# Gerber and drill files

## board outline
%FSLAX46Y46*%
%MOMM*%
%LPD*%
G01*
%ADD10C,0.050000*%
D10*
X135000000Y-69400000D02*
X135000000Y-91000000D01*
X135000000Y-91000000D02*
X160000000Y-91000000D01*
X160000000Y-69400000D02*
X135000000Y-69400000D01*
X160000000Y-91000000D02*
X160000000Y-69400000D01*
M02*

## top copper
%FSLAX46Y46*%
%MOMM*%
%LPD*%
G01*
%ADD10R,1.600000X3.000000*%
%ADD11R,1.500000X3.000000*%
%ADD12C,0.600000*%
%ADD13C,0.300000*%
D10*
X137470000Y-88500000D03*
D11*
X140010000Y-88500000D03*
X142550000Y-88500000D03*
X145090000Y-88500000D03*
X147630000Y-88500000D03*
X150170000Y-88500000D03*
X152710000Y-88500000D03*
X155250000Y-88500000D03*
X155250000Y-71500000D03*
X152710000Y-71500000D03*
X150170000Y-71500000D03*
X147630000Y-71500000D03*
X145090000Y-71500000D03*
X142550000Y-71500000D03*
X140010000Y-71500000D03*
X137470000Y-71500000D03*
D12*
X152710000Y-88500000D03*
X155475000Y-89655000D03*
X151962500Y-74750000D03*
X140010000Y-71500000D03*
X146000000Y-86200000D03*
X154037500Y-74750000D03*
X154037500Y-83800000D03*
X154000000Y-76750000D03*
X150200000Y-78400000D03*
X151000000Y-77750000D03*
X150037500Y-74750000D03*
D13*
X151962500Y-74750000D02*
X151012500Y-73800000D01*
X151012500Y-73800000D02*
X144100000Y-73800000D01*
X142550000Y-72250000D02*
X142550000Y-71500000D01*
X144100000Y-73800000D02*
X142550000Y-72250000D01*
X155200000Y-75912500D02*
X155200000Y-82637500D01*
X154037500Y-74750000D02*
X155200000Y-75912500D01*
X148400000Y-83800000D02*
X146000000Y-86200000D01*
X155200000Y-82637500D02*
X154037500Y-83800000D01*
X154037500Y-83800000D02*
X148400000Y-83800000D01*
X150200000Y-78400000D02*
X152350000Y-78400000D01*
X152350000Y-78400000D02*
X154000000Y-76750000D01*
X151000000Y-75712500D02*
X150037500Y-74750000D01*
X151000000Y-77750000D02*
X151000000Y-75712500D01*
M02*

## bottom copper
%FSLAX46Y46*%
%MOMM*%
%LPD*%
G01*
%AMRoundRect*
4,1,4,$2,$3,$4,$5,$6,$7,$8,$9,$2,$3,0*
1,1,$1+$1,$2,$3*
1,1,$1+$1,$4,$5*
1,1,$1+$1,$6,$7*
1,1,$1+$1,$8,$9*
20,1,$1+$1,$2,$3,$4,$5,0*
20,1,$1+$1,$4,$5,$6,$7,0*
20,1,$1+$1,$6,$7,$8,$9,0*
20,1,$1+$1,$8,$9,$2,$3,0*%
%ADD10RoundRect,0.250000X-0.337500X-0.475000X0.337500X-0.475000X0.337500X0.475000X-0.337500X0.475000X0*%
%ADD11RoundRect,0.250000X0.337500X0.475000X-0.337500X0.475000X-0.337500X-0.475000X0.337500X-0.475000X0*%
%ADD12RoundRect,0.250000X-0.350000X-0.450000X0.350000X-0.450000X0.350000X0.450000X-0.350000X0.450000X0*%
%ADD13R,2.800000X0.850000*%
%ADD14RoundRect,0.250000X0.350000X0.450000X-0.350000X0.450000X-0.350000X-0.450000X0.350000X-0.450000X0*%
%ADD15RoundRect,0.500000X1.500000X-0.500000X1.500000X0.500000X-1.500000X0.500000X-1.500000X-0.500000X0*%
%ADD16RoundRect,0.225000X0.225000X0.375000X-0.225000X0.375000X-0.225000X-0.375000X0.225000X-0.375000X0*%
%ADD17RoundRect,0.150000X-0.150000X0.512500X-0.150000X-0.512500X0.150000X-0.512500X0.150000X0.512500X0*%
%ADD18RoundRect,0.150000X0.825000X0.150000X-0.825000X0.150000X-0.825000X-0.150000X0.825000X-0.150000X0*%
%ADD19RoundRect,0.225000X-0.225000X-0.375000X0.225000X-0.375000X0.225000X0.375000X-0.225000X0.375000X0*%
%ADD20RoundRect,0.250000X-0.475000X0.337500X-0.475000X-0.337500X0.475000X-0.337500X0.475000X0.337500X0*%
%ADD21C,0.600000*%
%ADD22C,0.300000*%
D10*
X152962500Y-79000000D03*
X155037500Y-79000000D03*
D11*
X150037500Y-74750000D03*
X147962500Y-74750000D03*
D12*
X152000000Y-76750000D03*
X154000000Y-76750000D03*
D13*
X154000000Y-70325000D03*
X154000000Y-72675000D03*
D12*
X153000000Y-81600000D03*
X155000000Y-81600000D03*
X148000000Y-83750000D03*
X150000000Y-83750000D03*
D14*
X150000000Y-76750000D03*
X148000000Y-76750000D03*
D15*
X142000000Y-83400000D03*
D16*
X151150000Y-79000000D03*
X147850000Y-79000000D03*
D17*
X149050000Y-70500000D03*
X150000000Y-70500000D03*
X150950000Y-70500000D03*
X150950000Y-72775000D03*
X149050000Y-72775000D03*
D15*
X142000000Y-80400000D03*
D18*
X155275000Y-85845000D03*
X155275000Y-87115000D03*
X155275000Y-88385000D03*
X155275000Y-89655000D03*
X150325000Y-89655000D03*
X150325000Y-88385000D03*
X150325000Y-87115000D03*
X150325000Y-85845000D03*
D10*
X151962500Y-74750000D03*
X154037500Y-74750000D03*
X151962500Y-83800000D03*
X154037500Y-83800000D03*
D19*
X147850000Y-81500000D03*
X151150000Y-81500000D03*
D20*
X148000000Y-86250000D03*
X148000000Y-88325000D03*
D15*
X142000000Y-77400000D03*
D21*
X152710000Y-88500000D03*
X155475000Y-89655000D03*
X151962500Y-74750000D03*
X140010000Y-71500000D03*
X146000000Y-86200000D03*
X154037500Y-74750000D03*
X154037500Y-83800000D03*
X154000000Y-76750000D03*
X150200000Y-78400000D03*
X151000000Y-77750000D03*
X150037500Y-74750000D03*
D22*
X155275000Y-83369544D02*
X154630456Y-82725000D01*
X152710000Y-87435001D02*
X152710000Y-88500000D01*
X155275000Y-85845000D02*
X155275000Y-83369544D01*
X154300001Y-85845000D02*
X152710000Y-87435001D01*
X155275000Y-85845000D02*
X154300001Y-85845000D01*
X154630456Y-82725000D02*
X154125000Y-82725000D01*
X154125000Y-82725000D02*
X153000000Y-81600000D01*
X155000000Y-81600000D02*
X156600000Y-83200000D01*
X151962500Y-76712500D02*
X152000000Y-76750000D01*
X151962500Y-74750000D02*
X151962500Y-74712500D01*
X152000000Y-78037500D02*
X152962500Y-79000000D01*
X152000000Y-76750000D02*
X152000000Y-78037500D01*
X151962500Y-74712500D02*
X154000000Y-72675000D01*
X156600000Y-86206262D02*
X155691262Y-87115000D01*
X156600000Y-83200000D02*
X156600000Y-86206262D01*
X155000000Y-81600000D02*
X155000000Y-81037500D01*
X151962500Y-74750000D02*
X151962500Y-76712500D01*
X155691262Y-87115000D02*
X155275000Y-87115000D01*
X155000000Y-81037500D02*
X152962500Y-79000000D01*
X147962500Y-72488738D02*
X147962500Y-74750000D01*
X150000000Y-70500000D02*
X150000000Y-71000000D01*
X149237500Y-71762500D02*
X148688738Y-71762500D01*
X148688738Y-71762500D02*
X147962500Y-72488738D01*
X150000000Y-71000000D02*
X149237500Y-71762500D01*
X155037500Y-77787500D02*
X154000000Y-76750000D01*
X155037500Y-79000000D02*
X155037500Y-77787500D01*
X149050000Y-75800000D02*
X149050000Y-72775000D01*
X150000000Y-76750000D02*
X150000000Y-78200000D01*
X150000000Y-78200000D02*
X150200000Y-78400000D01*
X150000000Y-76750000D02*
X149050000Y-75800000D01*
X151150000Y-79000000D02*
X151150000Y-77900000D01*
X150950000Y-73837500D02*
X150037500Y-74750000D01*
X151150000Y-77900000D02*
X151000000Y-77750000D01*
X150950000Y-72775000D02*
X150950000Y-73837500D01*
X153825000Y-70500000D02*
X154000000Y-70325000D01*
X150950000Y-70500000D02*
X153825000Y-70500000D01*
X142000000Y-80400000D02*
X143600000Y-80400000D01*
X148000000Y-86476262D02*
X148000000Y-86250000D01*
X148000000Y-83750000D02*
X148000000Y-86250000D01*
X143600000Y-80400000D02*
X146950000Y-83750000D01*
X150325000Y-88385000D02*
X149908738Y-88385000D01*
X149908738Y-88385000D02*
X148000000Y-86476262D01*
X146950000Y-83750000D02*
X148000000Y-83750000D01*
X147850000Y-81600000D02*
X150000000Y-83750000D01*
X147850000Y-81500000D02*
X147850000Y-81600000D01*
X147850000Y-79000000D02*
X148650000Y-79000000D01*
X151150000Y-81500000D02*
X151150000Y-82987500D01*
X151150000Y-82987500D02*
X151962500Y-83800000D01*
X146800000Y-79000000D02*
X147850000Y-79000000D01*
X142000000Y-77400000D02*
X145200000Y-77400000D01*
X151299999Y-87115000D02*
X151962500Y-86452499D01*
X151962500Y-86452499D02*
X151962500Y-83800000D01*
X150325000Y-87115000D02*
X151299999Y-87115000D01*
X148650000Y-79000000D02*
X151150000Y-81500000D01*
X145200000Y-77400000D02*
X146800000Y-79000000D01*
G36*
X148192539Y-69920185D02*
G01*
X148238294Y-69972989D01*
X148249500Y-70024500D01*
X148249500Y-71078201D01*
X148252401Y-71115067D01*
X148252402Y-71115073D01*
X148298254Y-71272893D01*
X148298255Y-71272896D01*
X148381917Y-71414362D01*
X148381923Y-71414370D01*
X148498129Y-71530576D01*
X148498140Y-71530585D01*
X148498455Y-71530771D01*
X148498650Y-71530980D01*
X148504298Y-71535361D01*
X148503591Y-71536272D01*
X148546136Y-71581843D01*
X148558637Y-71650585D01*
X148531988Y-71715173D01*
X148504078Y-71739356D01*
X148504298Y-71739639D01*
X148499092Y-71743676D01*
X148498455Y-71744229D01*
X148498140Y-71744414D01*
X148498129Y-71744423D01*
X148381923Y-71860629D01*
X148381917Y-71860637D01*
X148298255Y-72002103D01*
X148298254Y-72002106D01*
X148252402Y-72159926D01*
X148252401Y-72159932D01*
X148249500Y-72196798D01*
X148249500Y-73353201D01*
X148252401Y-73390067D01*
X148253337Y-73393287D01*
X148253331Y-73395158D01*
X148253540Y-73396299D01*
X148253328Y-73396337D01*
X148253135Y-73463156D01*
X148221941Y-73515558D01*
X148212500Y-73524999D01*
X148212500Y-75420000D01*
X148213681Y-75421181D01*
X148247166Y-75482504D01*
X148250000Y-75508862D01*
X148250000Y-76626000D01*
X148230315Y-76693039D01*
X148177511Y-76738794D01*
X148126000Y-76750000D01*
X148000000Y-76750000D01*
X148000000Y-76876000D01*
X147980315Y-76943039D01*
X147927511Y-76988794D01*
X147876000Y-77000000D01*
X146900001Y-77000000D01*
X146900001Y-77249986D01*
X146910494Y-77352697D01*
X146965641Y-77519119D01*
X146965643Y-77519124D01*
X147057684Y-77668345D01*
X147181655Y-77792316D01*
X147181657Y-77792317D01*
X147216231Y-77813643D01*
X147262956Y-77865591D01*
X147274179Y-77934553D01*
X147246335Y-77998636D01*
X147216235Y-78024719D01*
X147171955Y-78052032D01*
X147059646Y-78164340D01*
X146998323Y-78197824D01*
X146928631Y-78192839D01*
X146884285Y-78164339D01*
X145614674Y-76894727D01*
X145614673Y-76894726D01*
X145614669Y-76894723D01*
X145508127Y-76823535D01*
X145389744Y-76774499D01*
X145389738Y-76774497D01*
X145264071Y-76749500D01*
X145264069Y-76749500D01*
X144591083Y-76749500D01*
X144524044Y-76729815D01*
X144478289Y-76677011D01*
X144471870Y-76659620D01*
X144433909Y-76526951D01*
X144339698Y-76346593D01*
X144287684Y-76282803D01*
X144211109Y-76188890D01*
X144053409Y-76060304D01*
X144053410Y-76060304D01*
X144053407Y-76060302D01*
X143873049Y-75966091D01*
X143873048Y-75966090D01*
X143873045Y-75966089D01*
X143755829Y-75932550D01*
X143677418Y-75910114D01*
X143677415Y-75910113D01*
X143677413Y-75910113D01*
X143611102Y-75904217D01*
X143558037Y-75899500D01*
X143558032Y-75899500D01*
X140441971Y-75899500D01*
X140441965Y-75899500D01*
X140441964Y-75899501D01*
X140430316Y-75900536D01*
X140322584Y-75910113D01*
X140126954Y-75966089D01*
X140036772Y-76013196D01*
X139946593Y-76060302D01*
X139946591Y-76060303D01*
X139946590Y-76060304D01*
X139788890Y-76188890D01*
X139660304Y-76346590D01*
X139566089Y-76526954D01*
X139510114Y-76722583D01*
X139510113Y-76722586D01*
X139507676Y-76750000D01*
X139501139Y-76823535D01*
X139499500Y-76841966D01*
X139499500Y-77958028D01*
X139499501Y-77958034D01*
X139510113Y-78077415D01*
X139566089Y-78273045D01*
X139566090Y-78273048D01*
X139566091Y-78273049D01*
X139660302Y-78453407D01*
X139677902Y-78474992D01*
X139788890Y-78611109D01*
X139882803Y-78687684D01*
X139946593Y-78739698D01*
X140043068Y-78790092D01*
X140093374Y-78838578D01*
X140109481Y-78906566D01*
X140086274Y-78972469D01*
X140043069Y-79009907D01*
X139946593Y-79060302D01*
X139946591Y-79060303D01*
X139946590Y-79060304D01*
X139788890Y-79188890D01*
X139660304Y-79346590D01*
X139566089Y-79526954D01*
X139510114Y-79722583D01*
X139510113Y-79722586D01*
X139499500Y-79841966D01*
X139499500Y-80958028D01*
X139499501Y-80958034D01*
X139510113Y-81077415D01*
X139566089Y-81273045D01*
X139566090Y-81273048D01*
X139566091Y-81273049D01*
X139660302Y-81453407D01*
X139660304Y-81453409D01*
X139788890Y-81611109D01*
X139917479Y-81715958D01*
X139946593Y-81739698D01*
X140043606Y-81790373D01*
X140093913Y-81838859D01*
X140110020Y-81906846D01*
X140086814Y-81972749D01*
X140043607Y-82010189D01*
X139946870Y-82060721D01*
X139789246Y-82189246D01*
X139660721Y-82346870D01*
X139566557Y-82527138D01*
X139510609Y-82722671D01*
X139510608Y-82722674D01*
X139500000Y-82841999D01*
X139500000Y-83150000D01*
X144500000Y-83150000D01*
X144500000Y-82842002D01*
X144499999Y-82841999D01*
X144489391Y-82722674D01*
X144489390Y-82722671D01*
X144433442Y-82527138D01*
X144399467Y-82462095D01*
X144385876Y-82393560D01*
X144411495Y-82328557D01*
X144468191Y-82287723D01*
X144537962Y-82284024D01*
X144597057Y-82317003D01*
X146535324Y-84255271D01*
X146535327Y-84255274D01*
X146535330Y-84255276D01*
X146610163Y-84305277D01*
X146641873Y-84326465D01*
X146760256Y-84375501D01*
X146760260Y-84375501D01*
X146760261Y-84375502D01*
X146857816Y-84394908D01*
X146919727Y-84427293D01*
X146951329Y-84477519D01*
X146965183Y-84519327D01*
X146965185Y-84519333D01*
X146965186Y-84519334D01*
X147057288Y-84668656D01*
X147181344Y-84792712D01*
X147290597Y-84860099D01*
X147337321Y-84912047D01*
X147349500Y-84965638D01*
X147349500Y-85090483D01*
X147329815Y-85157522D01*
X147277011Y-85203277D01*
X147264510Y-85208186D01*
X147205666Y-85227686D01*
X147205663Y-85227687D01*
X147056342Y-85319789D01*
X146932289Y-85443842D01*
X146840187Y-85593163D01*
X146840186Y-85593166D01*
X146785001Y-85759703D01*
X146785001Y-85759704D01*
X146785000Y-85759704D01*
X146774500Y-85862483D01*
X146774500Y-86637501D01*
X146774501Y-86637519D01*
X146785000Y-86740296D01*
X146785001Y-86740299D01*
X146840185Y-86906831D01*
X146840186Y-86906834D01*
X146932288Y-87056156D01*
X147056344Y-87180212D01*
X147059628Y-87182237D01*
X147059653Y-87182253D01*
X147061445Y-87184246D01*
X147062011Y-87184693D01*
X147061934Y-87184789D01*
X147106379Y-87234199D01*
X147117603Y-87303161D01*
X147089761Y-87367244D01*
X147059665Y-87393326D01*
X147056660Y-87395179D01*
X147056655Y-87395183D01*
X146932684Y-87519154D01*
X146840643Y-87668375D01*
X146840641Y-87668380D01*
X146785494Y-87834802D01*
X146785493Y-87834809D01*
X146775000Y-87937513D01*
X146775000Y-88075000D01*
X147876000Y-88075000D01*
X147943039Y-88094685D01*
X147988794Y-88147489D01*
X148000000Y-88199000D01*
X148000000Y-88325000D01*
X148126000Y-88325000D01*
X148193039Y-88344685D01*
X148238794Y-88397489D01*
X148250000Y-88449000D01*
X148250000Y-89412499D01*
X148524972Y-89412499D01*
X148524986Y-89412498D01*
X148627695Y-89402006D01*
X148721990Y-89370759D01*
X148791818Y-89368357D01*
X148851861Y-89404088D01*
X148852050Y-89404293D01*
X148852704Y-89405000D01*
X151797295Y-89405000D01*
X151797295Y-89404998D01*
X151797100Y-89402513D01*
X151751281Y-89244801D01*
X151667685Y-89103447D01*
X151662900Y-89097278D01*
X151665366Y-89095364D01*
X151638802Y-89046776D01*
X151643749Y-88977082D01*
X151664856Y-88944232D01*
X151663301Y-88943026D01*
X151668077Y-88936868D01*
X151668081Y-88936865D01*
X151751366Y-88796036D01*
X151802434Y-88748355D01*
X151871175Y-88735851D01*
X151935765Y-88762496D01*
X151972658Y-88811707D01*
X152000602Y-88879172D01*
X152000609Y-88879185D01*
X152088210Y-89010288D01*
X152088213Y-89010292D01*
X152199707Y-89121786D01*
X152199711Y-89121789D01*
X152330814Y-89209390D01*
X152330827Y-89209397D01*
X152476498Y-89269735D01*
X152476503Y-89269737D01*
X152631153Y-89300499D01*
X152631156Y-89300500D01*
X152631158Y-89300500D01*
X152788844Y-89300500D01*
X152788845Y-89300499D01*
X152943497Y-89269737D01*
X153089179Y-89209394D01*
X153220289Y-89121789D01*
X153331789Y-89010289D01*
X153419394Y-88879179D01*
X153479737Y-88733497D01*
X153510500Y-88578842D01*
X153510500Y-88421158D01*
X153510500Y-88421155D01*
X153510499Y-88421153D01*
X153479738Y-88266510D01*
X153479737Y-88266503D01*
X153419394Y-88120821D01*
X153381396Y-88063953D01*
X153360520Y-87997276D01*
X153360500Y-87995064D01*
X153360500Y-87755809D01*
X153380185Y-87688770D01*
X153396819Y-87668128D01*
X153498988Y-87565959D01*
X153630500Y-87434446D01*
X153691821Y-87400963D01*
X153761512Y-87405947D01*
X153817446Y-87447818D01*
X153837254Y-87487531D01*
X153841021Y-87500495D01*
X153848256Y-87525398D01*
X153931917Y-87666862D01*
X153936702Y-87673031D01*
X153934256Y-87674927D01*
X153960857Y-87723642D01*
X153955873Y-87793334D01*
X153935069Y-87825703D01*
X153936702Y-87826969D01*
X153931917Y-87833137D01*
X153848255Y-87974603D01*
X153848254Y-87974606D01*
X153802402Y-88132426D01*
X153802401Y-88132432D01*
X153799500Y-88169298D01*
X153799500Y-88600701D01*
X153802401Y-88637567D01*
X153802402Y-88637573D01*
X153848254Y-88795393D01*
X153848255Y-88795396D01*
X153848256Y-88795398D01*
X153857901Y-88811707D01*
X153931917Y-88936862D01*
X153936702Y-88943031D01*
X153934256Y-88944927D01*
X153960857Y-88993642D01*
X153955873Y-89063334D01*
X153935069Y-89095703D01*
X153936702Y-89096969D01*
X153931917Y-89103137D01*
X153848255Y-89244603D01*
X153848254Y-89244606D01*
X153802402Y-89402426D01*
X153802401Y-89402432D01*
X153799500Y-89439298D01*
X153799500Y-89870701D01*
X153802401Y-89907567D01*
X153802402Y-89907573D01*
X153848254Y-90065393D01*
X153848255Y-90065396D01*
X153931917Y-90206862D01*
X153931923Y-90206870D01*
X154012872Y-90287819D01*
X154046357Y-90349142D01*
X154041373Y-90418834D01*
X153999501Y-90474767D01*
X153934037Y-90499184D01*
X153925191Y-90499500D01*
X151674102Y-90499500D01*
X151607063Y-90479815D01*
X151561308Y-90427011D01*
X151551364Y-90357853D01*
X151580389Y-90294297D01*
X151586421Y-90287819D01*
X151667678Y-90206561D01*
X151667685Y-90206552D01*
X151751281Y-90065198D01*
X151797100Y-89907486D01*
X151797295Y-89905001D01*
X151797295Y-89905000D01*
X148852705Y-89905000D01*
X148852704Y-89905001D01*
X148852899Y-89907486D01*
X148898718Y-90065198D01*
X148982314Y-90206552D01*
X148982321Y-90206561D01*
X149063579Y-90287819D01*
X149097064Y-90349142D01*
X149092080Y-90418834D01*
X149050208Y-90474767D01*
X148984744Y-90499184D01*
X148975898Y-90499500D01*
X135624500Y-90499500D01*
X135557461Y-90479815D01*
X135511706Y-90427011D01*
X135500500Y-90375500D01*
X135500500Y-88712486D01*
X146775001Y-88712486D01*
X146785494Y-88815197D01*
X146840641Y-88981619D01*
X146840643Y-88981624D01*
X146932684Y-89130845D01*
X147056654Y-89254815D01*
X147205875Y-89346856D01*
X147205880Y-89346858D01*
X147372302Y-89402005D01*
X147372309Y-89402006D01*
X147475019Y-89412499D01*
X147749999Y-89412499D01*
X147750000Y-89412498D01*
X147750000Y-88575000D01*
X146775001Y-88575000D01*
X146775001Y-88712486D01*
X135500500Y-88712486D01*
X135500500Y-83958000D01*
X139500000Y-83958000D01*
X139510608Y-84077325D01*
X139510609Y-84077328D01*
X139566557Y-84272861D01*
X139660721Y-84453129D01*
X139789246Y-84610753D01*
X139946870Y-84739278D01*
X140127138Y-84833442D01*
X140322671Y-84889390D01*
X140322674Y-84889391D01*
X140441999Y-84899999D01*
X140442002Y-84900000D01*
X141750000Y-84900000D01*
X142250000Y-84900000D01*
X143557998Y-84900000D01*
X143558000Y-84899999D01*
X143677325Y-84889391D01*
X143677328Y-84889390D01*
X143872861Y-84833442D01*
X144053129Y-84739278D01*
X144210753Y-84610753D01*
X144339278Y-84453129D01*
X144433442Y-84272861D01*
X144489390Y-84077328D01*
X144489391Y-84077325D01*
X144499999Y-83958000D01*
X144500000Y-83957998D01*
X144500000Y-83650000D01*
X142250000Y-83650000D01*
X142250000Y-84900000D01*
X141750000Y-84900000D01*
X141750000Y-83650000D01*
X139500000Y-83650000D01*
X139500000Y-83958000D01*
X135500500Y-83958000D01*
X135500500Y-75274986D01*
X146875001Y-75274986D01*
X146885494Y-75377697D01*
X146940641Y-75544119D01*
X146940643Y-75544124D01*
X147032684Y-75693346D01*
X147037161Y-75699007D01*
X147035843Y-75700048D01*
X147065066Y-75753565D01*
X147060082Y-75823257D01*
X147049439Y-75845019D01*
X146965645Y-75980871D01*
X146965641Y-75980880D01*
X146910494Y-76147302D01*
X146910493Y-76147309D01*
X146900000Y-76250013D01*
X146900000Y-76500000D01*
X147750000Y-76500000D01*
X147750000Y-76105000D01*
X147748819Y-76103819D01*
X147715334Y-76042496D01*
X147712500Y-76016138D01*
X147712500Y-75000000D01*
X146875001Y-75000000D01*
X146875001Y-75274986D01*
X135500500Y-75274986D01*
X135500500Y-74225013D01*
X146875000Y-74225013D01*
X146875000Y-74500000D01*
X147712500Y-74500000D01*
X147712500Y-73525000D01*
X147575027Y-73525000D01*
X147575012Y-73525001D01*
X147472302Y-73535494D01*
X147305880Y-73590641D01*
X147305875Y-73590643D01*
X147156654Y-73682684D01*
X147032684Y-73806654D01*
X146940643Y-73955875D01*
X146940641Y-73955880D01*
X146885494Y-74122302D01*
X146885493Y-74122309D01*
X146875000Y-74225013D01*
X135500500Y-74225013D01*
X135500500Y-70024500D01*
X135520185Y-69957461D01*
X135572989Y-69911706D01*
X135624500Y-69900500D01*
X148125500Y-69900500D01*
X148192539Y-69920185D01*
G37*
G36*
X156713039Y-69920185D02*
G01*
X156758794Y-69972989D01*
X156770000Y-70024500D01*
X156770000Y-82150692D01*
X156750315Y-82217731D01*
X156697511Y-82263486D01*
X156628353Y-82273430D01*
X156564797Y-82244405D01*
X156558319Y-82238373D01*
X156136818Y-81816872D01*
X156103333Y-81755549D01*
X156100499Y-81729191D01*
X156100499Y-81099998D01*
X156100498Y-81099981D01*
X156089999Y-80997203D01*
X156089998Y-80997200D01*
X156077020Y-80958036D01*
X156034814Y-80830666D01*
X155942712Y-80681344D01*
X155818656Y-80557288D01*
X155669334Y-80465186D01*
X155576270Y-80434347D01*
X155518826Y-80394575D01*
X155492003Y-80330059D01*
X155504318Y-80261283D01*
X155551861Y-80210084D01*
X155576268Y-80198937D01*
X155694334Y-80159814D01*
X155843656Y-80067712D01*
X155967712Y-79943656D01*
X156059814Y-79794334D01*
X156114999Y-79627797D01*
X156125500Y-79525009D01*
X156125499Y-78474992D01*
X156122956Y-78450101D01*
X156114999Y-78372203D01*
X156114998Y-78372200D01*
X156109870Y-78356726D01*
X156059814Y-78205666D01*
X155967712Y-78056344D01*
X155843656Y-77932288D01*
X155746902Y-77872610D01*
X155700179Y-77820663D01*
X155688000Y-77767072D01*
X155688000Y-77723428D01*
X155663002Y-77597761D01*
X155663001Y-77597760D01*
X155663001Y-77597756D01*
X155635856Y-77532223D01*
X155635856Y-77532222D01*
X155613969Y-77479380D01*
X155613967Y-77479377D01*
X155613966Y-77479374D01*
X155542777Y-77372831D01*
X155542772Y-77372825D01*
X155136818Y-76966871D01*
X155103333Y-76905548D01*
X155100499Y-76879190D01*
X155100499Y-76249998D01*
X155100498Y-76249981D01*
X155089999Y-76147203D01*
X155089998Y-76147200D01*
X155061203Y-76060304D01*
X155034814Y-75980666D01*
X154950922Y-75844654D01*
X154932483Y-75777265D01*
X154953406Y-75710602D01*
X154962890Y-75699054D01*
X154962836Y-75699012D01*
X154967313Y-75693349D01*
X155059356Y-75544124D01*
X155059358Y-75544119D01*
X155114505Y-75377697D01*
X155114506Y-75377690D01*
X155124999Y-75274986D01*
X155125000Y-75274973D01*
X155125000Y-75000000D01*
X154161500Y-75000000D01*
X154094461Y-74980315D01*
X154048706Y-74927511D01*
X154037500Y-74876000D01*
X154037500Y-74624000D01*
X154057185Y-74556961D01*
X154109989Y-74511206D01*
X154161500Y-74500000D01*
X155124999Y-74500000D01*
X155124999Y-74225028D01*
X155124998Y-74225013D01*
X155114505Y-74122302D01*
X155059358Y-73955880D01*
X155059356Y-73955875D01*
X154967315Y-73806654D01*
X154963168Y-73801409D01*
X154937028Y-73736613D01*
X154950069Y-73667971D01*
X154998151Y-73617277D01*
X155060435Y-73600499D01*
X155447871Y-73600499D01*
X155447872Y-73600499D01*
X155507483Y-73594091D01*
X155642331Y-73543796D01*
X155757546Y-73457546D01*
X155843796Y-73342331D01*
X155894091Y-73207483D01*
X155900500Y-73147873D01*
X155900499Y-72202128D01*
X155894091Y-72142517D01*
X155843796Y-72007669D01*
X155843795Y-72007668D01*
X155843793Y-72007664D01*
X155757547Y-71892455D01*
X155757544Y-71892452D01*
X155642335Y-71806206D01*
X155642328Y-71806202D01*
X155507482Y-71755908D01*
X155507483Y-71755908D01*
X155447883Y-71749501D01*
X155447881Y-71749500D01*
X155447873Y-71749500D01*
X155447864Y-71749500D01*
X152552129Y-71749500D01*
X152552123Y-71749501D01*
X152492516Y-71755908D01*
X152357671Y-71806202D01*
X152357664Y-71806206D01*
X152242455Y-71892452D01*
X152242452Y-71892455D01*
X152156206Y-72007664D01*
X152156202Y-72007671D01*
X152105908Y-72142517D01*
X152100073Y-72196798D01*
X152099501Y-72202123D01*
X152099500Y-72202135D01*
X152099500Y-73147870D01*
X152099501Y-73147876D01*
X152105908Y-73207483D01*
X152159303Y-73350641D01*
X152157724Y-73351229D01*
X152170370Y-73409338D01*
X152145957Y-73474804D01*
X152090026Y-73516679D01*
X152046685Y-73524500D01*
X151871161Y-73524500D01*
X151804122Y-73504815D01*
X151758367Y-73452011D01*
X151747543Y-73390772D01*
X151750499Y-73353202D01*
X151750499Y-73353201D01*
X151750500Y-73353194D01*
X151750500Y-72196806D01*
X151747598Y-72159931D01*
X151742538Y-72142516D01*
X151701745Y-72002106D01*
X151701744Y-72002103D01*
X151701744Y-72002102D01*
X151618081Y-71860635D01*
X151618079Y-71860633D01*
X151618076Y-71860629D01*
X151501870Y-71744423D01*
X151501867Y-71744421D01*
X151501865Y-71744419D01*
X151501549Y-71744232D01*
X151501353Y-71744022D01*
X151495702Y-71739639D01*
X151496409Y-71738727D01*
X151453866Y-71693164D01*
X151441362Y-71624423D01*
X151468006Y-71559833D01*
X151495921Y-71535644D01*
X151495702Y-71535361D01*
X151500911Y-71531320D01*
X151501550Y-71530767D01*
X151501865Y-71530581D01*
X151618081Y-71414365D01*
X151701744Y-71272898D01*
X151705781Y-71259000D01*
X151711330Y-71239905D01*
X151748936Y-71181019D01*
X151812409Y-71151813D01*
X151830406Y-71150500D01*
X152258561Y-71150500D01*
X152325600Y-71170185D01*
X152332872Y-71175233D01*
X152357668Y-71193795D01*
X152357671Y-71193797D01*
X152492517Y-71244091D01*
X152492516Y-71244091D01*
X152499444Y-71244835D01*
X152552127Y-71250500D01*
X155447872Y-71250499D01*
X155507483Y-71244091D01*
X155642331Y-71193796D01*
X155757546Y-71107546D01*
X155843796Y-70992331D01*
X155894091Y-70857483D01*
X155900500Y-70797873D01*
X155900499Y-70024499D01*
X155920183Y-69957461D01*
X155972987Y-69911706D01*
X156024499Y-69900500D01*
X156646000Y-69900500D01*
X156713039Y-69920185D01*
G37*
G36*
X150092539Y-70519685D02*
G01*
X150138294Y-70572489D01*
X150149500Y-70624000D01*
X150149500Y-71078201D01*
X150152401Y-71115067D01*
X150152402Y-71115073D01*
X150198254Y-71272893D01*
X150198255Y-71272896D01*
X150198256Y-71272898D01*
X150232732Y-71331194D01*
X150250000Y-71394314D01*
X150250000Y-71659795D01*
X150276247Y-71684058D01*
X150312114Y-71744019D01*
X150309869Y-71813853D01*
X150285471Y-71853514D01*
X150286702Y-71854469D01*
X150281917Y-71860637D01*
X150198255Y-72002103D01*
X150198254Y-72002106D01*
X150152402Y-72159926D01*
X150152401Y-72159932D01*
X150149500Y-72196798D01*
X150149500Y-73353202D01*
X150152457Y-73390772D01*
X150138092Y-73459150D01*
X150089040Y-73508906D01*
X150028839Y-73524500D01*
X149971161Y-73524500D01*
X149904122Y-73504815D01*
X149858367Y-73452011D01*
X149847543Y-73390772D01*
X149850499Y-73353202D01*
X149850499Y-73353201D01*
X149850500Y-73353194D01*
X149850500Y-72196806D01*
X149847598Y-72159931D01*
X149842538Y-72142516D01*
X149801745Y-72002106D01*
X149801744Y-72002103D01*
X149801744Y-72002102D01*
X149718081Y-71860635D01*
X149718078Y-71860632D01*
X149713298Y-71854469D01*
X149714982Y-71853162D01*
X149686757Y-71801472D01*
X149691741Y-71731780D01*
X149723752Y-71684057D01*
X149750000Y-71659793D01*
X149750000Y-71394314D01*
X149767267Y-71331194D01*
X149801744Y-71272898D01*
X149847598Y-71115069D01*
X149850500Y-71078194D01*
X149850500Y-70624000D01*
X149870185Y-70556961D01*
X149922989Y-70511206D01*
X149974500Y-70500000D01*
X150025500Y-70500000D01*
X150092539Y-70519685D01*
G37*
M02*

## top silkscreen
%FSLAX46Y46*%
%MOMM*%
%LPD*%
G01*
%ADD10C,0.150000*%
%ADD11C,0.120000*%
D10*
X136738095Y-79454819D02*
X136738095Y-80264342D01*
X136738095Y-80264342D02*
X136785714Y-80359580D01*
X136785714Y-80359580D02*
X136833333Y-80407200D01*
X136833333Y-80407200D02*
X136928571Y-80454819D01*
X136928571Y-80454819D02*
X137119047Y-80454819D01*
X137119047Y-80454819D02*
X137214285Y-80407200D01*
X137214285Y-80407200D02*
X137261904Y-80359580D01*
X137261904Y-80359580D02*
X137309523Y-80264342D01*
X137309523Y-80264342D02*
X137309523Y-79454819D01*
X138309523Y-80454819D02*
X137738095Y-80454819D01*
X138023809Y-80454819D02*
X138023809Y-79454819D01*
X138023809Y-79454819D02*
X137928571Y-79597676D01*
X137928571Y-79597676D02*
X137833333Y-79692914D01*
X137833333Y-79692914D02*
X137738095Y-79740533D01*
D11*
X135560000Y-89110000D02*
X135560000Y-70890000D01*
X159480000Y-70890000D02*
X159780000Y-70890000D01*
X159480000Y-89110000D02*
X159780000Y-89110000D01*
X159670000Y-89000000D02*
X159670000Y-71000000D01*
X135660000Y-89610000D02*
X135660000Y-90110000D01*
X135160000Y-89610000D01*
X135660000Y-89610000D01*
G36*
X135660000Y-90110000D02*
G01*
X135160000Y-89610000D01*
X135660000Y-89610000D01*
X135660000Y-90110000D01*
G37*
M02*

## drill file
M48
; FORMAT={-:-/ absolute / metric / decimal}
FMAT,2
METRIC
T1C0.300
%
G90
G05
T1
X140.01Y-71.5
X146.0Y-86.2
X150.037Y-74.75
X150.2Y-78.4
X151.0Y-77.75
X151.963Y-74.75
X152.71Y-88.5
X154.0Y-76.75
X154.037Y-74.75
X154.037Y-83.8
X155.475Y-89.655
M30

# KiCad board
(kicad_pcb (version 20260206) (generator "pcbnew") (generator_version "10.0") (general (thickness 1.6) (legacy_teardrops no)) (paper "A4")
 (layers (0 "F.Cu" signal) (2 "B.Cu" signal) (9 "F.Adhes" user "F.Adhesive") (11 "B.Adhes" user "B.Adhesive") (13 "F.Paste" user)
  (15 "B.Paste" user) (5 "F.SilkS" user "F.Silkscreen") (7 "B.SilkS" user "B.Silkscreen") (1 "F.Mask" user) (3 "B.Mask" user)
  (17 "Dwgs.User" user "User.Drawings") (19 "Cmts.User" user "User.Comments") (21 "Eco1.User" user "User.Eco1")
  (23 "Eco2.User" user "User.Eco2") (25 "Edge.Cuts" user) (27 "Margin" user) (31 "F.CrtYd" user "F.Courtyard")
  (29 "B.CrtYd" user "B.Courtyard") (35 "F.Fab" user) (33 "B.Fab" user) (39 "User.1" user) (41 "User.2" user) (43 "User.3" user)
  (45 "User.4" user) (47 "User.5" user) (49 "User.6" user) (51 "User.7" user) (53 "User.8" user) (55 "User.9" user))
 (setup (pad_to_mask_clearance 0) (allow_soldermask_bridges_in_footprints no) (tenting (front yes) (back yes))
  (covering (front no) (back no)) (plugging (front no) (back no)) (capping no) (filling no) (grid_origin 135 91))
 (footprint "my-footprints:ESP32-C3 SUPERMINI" (layer "F.Cu") (at 152.47 80 90)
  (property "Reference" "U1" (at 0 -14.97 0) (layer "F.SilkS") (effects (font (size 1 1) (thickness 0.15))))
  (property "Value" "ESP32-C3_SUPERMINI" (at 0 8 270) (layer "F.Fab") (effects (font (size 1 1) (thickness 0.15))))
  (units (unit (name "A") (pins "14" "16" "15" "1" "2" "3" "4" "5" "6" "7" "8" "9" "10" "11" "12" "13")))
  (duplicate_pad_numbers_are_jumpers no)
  (fp_line (start -9.11 -16.91) (end 9.11 -16.91) (stroke (width 0.12) (type solid)) (layer "F.SilkS"))
  (fp_line (start 9.11 7.01) (end 9.11 7.31) (stroke (width 0.12) (type solid)) (layer "F.SilkS"))
  (fp_line (start -9.11 7.01) (end -9.11 7.31) (stroke (width 0.12) (type solid)) (layer "F.SilkS"))
  (fp_line (start -9 7.2) (end 9 7.2) (stroke (width 0.12) (type solid)) (layer "F.SilkS"))
  (fp_poly
   (pts (xy -9.61 -16.81) (xy -10.11 -16.81) (xy -9.61 -17.31) (xy -9.61 -16.81)) (stroke (width 0.12) (type solid)) (fill yes)
   (layer "F.SilkS"))
  (pad "1" smd rect (at -8.5 -15 90) (size 3 1.6) (layers "F.Cu" "F.Mask" "F.Paste") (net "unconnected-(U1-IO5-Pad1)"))
  (pad "2" smd rect (at -8.5 -12.46 90) (size 3 1.5) (layers "F.Cu" "F.Mask" "F.Paste") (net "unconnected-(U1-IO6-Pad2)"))
  (pad "3" smd rect (at -8.5 -9.92 90) (size 3 1.5) (layers "F.Cu" "F.Mask" "F.Paste") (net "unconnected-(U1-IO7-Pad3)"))
  (pad "4" smd rect (at -8.5 -7.38 90) (size 3 1.5) (layers "F.Cu" "F.Mask" "F.Paste") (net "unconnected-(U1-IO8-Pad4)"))
  (pad "5" smd rect (at -8.5 -4.84 90) (size 3 1.5) (layers "F.Cu" "F.Mask" "F.Paste") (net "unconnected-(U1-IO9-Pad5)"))
  (pad "6" smd rect (at -8.5 -2.3 90) (size 3 1.5) (layers "F.Cu" "F.Mask" "F.Paste") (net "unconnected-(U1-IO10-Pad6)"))
  (pad "7" smd rect (at -8.5 0.24 90) (size 3 1.5) (layers "F.Cu" "F.Mask" "F.Paste") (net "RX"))
  (pad "8" smd rect (at -8.5 2.78 90) (size 3 1.5) (layers "F.Cu" "F.Mask" "F.Paste") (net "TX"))
  (pad "9" smd rect (at 8.5 2.78 90) (size 3 1.5) (layers "F.Cu" "F.Mask" "F.Paste") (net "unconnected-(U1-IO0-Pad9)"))
  (pad "10" smd rect (at 8.5 0.24 90) (size 3 1.5) (layers "F.Cu" "F.Mask" "F.Paste") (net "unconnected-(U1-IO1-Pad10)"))
  (pad "11" smd rect (at 8.5 -2.3 90) (size 3 1.5) (layers "F.Cu" "F.Mask" "F.Paste") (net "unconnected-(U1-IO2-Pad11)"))
  (pad "12" smd rect (at 8.5 -4.84 90) (size 3 1.5) (layers "F.Cu" "F.Mask" "F.Paste") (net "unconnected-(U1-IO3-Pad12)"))
  (pad "13" smd rect (at 8.5 -7.38 90) (size 3 1.5) (layers "F.Cu" "F.Mask" "F.Paste") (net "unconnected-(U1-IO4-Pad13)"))
  (pad "14" smd rect (at 8.5 -9.92 90) (size 3 1.5) (layers "F.Cu" "F.Mask" "F.Paste") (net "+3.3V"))
  (pad "15" smd rect (at 8.5 -12.46 90) (size 3 1.5) (layers "F.Cu" "F.Mask" "F.Paste") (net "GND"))
  (pad "16" smd rect (at 8.5 -15 90) (size 3 1.5) (layers "F.Cu" "F.Mask" "F.Paste") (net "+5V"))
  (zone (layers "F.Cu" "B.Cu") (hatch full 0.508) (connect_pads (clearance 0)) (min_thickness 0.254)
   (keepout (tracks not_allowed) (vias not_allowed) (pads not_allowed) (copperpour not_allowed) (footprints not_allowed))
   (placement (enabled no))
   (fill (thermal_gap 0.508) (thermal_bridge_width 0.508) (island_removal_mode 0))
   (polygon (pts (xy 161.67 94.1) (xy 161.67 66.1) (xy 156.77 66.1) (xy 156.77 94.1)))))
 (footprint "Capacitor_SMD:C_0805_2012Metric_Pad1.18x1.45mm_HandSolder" (layer "B.Cu") (at 154 79)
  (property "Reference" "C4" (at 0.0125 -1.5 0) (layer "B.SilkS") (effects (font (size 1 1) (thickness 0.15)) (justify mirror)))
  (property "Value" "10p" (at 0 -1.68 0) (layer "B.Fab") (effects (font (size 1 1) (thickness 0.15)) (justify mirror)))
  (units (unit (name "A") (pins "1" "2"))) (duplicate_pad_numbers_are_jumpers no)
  (pad "1" smd roundrect (at -1.0375 0) (size 1.175 1.45) (layers "B.Cu" "B.Mask" "B.Paste") (roundrect_rratio 0.212766) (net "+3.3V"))
  (pad "2" smd roundrect (at 1.0375 0) (size 1.175 1.45) (layers "B.Cu" "B.Mask" "B.Paste") (roundrect_rratio 0.212766) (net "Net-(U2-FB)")))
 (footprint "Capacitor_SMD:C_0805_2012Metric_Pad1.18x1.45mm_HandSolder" (layer "B.Cu") (at 149 74.75 180)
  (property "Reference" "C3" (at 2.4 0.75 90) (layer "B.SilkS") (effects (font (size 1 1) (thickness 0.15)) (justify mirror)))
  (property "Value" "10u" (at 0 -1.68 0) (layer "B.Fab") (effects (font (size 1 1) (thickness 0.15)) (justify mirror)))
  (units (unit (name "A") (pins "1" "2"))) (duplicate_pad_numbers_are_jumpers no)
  (pad "1" smd roundrect (at -1.0375 0 180) (size 1.175 1.45) (layers "B.Cu" "B.Mask" "B.Paste") (roundrect_rratio 0.212766)
   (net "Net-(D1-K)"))
  (pad "2" smd roundrect (at 1.0375 0 180) (size 1.175 1.45) (layers "B.Cu" "B.Mask" "B.Paste") (roundrect_rratio 0.212766) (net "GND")))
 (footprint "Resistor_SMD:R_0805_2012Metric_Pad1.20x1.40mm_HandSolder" (layer "B.Cu") (at 153 76.75)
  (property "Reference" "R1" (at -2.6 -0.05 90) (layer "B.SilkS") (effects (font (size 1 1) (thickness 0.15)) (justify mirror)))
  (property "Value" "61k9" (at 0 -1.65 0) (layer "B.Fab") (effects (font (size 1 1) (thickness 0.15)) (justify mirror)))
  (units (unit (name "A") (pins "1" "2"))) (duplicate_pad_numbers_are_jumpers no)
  (pad "1" smd roundrect (at -1 0) (size 1.2 1.4) (layers "B.Cu" "B.Mask" "B.Paste") (roundrect_rratio 0.208333) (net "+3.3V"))
  (pad "2" smd roundrect (at 1 0) (size 1.2 1.4) (layers "B.Cu" "B.Mask" "B.Paste") (roundrect_rratio 0.208333) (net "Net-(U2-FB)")))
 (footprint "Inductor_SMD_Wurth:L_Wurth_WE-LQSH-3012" (layer "B.Cu") (at 154 71.5 -90)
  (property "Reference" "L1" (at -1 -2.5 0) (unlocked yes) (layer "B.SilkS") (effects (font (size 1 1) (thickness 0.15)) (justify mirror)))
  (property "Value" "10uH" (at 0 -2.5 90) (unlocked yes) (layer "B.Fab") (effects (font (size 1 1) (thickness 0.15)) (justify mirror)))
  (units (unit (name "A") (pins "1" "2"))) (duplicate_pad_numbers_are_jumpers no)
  (pad "1" smd rect (at -1.175 0 270) (size 0.85 2.8) (layers "B.Cu" "B.Mask" "B.Paste") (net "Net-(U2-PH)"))
  (pad "2" smd rect (at 1.175 0 270) (size 0.85 2.8) (layers "B.Cu" "B.Mask" "B.Paste") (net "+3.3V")))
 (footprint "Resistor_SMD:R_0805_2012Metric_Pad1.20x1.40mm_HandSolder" (layer "B.Cu") (at 154 81.6)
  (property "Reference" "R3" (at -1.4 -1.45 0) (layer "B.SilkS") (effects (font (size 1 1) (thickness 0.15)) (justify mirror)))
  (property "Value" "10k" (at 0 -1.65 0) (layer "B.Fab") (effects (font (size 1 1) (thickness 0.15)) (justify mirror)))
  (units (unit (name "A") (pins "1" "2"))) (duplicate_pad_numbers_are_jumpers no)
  (pad "1" smd roundrect (at -1 0) (size 1.2 1.4) (layers "B.Cu" "B.Mask" "B.Paste") (roundrect_rratio 0.208333) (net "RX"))
  (pad "2" smd roundrect (at 1 0) (size 1.2 1.4) (layers "B.Cu" "B.Mask" "B.Paste") (roundrect_rratio 0.208333) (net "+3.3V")))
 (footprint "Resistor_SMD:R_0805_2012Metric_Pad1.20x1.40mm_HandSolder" (layer "B.Cu") (at 149 83.75)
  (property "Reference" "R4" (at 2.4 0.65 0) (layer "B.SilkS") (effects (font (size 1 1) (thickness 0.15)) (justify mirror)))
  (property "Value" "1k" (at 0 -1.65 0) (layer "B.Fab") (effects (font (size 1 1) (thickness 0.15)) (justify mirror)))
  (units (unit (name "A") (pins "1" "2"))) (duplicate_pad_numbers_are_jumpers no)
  (pad "1" smd roundrect (at -1 0) (size 1.2 1.4) (layers "B.Cu" "B.Mask" "B.Paste") (roundrect_rratio 0.208333) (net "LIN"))
  (pad "2" smd roundrect (at 1 0) (size 1.2 1.4) (layers "B.Cu" "B.Mask" "B.Paste") (roundrect_rratio 0.208333) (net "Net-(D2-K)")))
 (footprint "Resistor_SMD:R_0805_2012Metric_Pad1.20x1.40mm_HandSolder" (layer "B.Cu") (at 149 76.75 180)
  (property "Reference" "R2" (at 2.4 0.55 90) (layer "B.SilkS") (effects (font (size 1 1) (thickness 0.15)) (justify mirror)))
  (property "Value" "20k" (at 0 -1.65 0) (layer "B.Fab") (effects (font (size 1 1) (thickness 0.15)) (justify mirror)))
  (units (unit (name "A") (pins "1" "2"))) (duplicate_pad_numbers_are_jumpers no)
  (pad "1" smd roundrect (at -1 0 180) (size 1.2 1.4) (layers "B.Cu" "B.Mask" "B.Paste") (roundrect_rratio 0.208333) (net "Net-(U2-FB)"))
  (pad "2" smd roundrect (at 1 0 180) (size 1.2 1.4) (layers "B.Cu" "B.Mask" "B.Paste") (roundrect_rratio 0.208333) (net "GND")))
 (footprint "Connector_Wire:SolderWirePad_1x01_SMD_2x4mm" (layer "B.Cu") (at 142 83.4 90)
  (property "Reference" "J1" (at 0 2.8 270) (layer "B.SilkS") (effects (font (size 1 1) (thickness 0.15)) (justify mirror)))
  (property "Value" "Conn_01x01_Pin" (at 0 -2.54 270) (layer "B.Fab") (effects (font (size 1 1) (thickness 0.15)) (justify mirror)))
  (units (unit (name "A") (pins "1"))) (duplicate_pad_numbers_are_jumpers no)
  (pad "1" smd roundrect (at 0 0 90) (size 2 4) (layers "B.Cu" "B.Mask") (roundrect_rratio 0.25) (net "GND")))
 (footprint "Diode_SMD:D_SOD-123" (layer "B.Cu") (at 149.5 79 180)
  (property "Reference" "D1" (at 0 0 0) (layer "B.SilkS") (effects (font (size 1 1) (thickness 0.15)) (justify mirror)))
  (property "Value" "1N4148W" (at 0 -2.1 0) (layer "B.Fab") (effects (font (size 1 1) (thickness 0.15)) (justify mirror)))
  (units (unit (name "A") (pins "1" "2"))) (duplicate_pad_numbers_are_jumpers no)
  (pad "1" smd roundrect (at -1.65 0 180) (size 0.9 1.2) (layers "B.Cu" "B.Mask" "B.Paste") (roundrect_rratio 0.25) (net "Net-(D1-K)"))
  (pad "2" smd roundrect (at 1.65 0 180) (size 0.9 1.2) (layers "B.Cu" "B.Mask" "B.Paste") (roundrect_rratio 0.25) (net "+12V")))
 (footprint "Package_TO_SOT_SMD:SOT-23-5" (layer "B.Cu") (at 150 71.6375 -90)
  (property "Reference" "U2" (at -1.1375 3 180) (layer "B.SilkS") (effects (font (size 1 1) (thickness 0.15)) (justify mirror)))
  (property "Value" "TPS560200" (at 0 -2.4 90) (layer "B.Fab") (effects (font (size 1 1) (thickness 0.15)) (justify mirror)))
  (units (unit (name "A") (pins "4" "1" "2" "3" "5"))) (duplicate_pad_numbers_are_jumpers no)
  (pad "1" smd roundrect (at -1.1375 0.95 270) (size 1.325 0.6) (layers "B.Cu" "B.Mask" "B.Paste") (roundrect_rratio 0.25)
   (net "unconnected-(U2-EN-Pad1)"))
  (pad "2" smd roundrect (at -1.1375 0 270) (size 1.325 0.6) (layers "B.Cu" "B.Mask" "B.Paste") (roundrect_rratio 0.25) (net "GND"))
  (pad "3" smd roundrect (at -1.1375 -0.95 270) (size 1.325 0.6) (layers "B.Cu" "B.Mask" "B.Paste") (roundrect_rratio 0.25)
   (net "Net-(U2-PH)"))
  (pad "4" smd roundrect (at 1.1375 -0.95 270) (size 1.325 0.6) (layers "B.Cu" "B.Mask" "B.Paste") (roundrect_rratio 0.25)
   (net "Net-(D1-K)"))
  (pad "5" smd roundrect (at 1.1375 0.95 270) (size 1.325 0.6) (layers "B.Cu" "B.Mask" "B.Paste") (roundrect_rratio 0.25)
   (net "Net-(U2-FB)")))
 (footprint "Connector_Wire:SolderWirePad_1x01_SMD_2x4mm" (layer "B.Cu") (at 142 80.4 90)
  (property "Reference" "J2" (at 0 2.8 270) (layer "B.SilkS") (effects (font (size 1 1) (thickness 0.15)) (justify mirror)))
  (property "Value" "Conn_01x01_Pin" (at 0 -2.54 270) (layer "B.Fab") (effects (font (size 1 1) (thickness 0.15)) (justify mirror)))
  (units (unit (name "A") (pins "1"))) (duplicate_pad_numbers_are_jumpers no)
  (pad "1" smd roundrect (at 0 0 90) (size 2 4) (layers "B.Cu" "B.Mask") (roundrect_rratio 0.25) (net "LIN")))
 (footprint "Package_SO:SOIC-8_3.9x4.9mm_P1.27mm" (layer "B.Cu") (at 152.8 87.75 180)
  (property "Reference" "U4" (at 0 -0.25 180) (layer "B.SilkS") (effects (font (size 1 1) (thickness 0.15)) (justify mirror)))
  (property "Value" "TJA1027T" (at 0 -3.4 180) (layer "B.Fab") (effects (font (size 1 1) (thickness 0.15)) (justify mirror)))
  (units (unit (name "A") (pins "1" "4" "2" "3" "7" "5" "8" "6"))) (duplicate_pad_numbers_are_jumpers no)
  (pad "1" smd roundrect (at -2.475 1.905 180) (size 1.95 0.6) (layers "B.Cu" "B.Mask" "B.Paste") (roundrect_rratio 0.25) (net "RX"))
  (pad "2" smd roundrect (at -2.475 0.635 180) (size 1.95 0.6) (layers "B.Cu" "B.Mask" "B.Paste") (roundrect_rratio 0.25) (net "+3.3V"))
  (pad "3" smd roundrect (at -2.475 -0.635 180) (size 1.95 0.6) (layers "B.Cu" "B.Mask" "B.Paste") (roundrect_rratio 0.25)
   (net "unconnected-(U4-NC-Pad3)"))
  (pad "4" smd roundrect (at -2.475 -1.905 180) (size 1.95 0.6) (layers "B.Cu" "B.Mask" "B.Paste") (roundrect_rratio 0.25) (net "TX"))
  (pad "5" smd roundrect (at 2.475 -1.905 180) (size 1.95 0.6) (layers "B.Cu" "B.Mask" "B.Paste") (roundrect_rratio 0.25) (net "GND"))
  (pad "6" smd roundrect (at 2.475 -0.635 180) (size 1.95 0.6) (layers "B.Cu" "B.Mask" "B.Paste") (roundrect_rratio 0.25) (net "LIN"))
  (pad "7" smd roundrect (at 2.475 0.635 180) (size 1.95 0.6) (layers "B.Cu" "B.Mask" "B.Paste") (roundrect_rratio 0.25) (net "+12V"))
  (pad "8" smd roundrect (at 2.475 1.905 180) (size 1.95 0.6) (layers "B.Cu" "B.Mask" "B.Paste") (roundrect_rratio 0.25)
   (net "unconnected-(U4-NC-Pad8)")))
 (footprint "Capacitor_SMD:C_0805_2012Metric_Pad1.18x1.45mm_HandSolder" (layer "B.Cu") (at 153 74.75)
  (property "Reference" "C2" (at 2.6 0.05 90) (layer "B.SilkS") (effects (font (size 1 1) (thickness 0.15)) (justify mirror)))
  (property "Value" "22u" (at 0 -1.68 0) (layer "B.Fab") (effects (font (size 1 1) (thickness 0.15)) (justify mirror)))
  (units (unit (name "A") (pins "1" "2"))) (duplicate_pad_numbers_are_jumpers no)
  (pad "1" smd roundrect (at -1.0375 0) (size 1.175 1.45) (layers "B.Cu" "B.Mask" "B.Paste") (roundrect_rratio 0.212766) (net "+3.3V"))
  (pad "2" smd roundrect (at 1.0375 0) (size 1.175 1.45) (layers "B.Cu" "B.Mask" "B.Paste") (roundrect_rratio 0.212766) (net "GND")))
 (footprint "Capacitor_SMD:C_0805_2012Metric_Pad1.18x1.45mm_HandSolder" (layer "B.Cu") (at 153 83.8)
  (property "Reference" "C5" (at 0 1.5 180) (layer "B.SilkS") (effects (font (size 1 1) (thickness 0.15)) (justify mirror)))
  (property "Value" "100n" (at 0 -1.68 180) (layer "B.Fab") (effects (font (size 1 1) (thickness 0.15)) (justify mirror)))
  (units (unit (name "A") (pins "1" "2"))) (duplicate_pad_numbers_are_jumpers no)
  (pad "1" smd roundrect (at -1.0375 0) (size 1.175 1.45) (layers "B.Cu" "B.Mask" "B.Paste") (roundrect_rratio 0.212766) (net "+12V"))
  (pad "2" smd roundrect (at 1.0375 0) (size 1.175 1.45) (layers "B.Cu" "B.Mask" "B.Paste") (roundrect_rratio 0.212766) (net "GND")))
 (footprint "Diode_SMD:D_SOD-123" (layer "B.Cu") (at 149.5 81.5)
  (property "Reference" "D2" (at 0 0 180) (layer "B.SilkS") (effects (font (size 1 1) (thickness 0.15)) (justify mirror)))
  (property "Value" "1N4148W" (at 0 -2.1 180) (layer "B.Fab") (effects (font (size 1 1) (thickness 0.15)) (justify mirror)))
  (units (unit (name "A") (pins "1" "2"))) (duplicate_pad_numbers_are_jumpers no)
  (pad "1" smd roundrect (at -1.65 0) (size 0.9 1.2) (layers "B.Cu" "B.Mask" "B.Paste") (roundrect_rratio 0.25) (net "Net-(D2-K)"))
  (pad "2" smd roundrect (at 1.65 0) (size 0.9 1.2) (layers "B.Cu" "B.Mask" "B.Paste") (roundrect_rratio 0.25) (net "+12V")))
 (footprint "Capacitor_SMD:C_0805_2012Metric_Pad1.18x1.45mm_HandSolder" (layer "B.Cu") (at 148 87.2875 -90)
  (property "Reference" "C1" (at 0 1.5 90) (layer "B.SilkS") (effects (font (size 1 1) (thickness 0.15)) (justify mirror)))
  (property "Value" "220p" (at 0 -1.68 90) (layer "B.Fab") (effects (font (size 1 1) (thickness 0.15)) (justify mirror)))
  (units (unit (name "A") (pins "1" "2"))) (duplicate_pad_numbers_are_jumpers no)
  (pad "1" smd roundrect (at -1.0375 0 270) (size 1.175 1.45) (layers "B.Cu" "B.Mask" "B.Paste") (roundrect_rratio 0.212766) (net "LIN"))
  (pad "2" smd roundrect (at 1.0375 0 270) (size 1.175 1.45) (layers "B.Cu" "B.Mask" "B.Paste") (roundrect_rratio 0.212766) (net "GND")))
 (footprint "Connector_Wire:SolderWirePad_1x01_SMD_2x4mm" (layer "B.Cu") (at 142 77.4 90)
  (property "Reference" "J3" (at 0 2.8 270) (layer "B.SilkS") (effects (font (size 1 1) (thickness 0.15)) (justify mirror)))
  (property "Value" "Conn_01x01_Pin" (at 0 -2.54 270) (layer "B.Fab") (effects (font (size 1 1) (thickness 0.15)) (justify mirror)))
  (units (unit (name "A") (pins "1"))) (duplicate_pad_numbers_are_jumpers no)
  (pad "1" smd roundrect (at 0 0 90) (size 2 4) (layers "B.Cu" "B.Mask") (roundrect_rratio 0.25) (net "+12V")))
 (gr_line (start 135 69.4) (end 135 91) (stroke (width 0.05) (type default)) (layer "Edge.Cuts"))
 (gr_line (start 135 91) (end 160 91) (stroke (width 0.05) (type default)) (layer "Edge.Cuts"))
 (gr_line (start 160 69.4) (end 135 69.4) (stroke (width 0.05) (type default)) (layer "Edge.Cuts"))
 (gr_line (start 160 91) (end 160 69.4) (stroke (width 0.05) (type default)) (layer "Edge.Cuts"))
 (via (at 152.71 88.5) (size 0.6) (drill 0.3) (layers "F.Cu" "B.Cu") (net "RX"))
 (segment (start 155.275 83.369544) (end 154.630456 82.725) (width 0.3) (layer "B.Cu") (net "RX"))
 (segment (start 152.71 87.435001) (end 152.71 88.5) (width 0.3) (layer "B.Cu") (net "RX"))
 (segment (start 155.275 85.845) (end 155.275 83.369544) (width 0.3) (layer "B.Cu") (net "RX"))
 (segment (start 154.300001 85.845) (end 152.71 87.435001) (width 0.3) (layer "B.Cu") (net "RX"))
 (segment (start 155.275 85.845) (end 154.300001 85.845) (width 0.3) (layer "B.Cu") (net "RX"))
 (segment (start 154.630456 82.725) (end 154.125 82.725) (width 0.3) (layer "B.Cu") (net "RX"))
 (segment (start 154.125 82.725) (end 153 81.6) (width 0.3) (layer "B.Cu") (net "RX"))
 (via (at 155.475 89.655) (size 0.6) (drill 0.3) (layers "F.Cu" "B.Cu") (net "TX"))
 (segment (start 151.9625 74.75) (end 151.0125 73.8) (width 0.3) (layer "F.Cu") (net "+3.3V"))
 (segment (start 151.0125 73.8) (end 144.1 73.8) (width 0.3) (layer "F.Cu") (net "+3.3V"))
 (segment (start 142.55 72.25) (end 142.55 71.5) (width 0.3) (layer "F.Cu") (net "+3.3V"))
 (segment (start 144.1 73.8) (end 142.55 72.25) (width 0.3) (layer "F.Cu") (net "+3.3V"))
 (via (at 151.9625 74.75) (size 0.6) (drill 0.3) (layers "F.Cu" "B.Cu") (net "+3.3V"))
 (segment (start 155 81.6) (end 156.6 83.2) (width 0.3) (layer "B.Cu") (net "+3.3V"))
 (segment (start 151.9625 76.7125) (end 152 76.75) (width 0.3) (layer "B.Cu") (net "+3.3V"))
 (segment (start 151.9625 74.75) (end 151.9625 74.7125) (width 0.3) (layer "B.Cu") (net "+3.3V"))
 (segment (start 152 78.0375) (end 152.9625 79) (width 0.3) (layer "B.Cu") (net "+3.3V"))
 (segment (start 152 76.75) (end 152 78.0375) (width 0.3) (layer "B.Cu") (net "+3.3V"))
 (segment (start 151.9625 74.7125) (end 154 72.675) (width 0.3) (layer "B.Cu") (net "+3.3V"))
 (segment (start 156.6 86.206262) (end 155.691262 87.115) (width 0.3) (layer "B.Cu") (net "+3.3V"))
 (segment (start 156.6 83.2) (end 156.6 86.206262) (width 0.3) (layer "B.Cu") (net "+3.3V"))
 (segment (start 155 81.6) (end 155 81.0375) (width 0.3) (layer "B.Cu") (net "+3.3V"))
 (segment (start 151.9625 74.75) (end 151.9625 76.7125) (width 0.3) (layer "B.Cu") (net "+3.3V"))
 (segment (start 155.691262 87.115) (end 155.275 87.115) (width 0.3) (layer "B.Cu") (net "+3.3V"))
 (segment (start 155 81.0375) (end 152.9625 79) (width 0.3) (layer "B.Cu") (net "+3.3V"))
 (segment (start 155.2 75.9125) (end 155.2 82.6375) (width 0.3) (layer "F.Cu") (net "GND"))
 (segment (start 154.0375 74.75) (end 155.2 75.9125) (width 0.3) (layer "F.Cu") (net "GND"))
 (segment (start 148.4 83.8) (end 146 86.2) (width 0.3) (layer "F.Cu") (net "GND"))
 (segment (start 155.2 82.6375) (end 154.0375 83.8) (width 0.3) (layer "F.Cu") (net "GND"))
 (segment (start 154.0375 83.8) (end 148.4 83.8) (width 0.3) (layer "F.Cu") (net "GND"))
 (via (at 140.01 71.5) (size 0.6) (drill 0.3) (layers "F.Cu" "B.Cu") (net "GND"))
 (via (at 146 86.2) (size 0.6) (drill 0.3) (layers "F.Cu" "B.Cu") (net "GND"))
 (via (at 154.0375 74.75) (size 0.6) (drill 0.3) (layers "F.Cu" "B.Cu") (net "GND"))
 (via (at 154.0375 83.8) (size 0.6) (drill 0.3) (layers "F.Cu" "B.Cu") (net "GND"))
 (segment (start 147.9625 72.488738) (end 147.9625 74.75) (width 0.3) (layer "B.Cu") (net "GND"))
 (segment (start 150 70.5) (end 150 71) (width 0.3) (layer "B.Cu") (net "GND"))
 (segment (start 149.2375 71.7625) (end 148.688738 71.7625) (width 0.3) (layer "B.Cu") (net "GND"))
 (segment (start 148.688738 71.7625) (end 147.9625 72.488738) (width 0.3) (layer "B.Cu") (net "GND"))
 (segment (start 150 71) (end 149.2375 71.7625) (width 0.3) (layer "B.Cu") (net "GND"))
 (segment (start 150.2 78.4) (end 152.35 78.4) (width 0.3) (layer "F.Cu") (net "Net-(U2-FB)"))
 (segment (start 152.35 78.4) (end 154 76.75) (width 0.3) (layer "F.Cu") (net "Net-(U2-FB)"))
 (via (at 154 76.75) (size 0.6) (drill 0.3) (layers "F.Cu" "B.Cu") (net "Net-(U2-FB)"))
 (via (at 150.2 78.4) (size 0.6) (drill 0.3) (layers "F.Cu" "B.Cu") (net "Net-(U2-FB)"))
 (segment (start 155.0375 77.7875) (end 154 76.75) (width 0.3) (layer "B.Cu") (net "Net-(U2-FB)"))
 (segment (start 155.0375 79) (end 155.0375 77.7875) (width 0.3) (layer "B.Cu") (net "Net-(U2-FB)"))
 (segment (start 149.05 75.8) (end 149.05 72.775) (width 0.3) (layer "B.Cu") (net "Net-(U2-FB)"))
 (segment (start 150 76.75) (end 150 78.2) (width 0.3) (layer "B.Cu") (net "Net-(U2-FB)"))
 (segment (start 150 78.2) (end 150.2 78.4) (width 0.3) (layer "B.Cu") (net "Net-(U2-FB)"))
 (segment (start 150 76.75) (end 149.05 75.8) (width 0.3) (layer "B.Cu") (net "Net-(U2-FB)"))
 (segment (start 151 75.7125) (end 150.0375 74.75) (width 0.3) (layer "F.Cu") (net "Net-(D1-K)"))
 (segment (start 151 77.75) (end 151 75.7125) (width 0.3) (layer "F.Cu") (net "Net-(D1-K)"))
 (via (at 151 77.75) (size 0.6) (drill 0.3) (layers "F.Cu" "B.Cu") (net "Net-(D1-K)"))
 (via (at 150.0375 74.75) (size 0.6) (drill 0.3) (layers "F.Cu" "B.Cu") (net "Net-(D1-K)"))
 (segment (start 151.15 79) (end 151.15 77.9) (width 0.3) (layer "B.Cu") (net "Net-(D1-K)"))
 (segment (start 150.95 73.8375) (end 150.0375 74.75) (width 0.3) (layer "B.Cu") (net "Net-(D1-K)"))
 (segment (start 151.15 77.9) (end 151 77.75) (width 0.3) (layer "B.Cu") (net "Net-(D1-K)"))
 (segment (start 150.95 72.775) (end 150.95 73.8375) (width 0.3) (layer "B.Cu") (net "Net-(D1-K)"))
 (segment (start 153.825 70.5) (end 154 70.325) (width 0.3) (layer "B.Cu") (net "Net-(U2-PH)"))
 (segment (start 150.95 70.5) (end 153.825 70.5) (width 0.3) (layer "B.Cu") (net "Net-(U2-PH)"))
 (segment (start 142 80.4) (end 143.6 80.4) (width 0.3) (layer "B.Cu") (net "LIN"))
 (segment (start 148 86.476262) (end 148 86.25) (width 0.3) (layer "B.Cu") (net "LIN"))
 (segment (start 148 83.75) (end 148 86.25) (width 0.3) (layer "B.Cu") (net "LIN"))
 (segment (start 143.6 80.4) (end 146.95 83.75) (width 0.3) (layer "B.Cu") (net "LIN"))
 (segment (start 150.325 88.385) (end 149.908738 88.385) (width 0.3) (layer "B.Cu") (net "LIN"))
 (segment (start 149.908738 88.385) (end 148 86.476262) (width 0.3) (layer "B.Cu") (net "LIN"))
 (segment (start 146.95 83.75) (end 148 83.75) (width 0.3) (layer "B.Cu") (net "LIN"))
 (segment (start 147.85 81.6) (end 150 83.75) (width 0.3) (layer "B.Cu") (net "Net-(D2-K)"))
 (segment (start 147.85 81.5) (end 147.85 81.6) (width 0.3) (layer "B.Cu") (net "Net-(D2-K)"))
 (segment (start 147.85 79) (end 148.65 79) (width 0.3) (layer "B.Cu") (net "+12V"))
 (segment (start 151.15 81.5) (end 151.15 82.9875) (width 0.3) (layer "B.Cu") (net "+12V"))
 (segment (start 151.15 82.9875) (end 151.9625 83.8) (width 0.3) (layer "B.Cu") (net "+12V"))
 (segment (start 146.8 79) (end 147.85 79) (width 0.3) (layer "B.Cu") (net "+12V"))
 (segment (start 142 77.4) (end 145.2 77.4) (width 0.3) (layer "B.Cu") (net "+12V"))
 (segment (start 151.299999 87.115) (end 151.9625 86.452499) (width 0.3) (layer "B.Cu") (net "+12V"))
 (segment (start 151.9625 86.452499) (end 151.9625 83.8) (width 0.3) (layer "B.Cu") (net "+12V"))
 (segment (start 150.325 87.115) (end 151.299999 87.115) (width 0.3) (layer "B.Cu") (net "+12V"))
 (segment (start 148.65 79) (end 151.15 81.5) (width 0.3) (layer "B.Cu") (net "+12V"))
 (segment (start 145.2 77.4) (end 146.8 79) (width 0.3) (layer "B.Cu") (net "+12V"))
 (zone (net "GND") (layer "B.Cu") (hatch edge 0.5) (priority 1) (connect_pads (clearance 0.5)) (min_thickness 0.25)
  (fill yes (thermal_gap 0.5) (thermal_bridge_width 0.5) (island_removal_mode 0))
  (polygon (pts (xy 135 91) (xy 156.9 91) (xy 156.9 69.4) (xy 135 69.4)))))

